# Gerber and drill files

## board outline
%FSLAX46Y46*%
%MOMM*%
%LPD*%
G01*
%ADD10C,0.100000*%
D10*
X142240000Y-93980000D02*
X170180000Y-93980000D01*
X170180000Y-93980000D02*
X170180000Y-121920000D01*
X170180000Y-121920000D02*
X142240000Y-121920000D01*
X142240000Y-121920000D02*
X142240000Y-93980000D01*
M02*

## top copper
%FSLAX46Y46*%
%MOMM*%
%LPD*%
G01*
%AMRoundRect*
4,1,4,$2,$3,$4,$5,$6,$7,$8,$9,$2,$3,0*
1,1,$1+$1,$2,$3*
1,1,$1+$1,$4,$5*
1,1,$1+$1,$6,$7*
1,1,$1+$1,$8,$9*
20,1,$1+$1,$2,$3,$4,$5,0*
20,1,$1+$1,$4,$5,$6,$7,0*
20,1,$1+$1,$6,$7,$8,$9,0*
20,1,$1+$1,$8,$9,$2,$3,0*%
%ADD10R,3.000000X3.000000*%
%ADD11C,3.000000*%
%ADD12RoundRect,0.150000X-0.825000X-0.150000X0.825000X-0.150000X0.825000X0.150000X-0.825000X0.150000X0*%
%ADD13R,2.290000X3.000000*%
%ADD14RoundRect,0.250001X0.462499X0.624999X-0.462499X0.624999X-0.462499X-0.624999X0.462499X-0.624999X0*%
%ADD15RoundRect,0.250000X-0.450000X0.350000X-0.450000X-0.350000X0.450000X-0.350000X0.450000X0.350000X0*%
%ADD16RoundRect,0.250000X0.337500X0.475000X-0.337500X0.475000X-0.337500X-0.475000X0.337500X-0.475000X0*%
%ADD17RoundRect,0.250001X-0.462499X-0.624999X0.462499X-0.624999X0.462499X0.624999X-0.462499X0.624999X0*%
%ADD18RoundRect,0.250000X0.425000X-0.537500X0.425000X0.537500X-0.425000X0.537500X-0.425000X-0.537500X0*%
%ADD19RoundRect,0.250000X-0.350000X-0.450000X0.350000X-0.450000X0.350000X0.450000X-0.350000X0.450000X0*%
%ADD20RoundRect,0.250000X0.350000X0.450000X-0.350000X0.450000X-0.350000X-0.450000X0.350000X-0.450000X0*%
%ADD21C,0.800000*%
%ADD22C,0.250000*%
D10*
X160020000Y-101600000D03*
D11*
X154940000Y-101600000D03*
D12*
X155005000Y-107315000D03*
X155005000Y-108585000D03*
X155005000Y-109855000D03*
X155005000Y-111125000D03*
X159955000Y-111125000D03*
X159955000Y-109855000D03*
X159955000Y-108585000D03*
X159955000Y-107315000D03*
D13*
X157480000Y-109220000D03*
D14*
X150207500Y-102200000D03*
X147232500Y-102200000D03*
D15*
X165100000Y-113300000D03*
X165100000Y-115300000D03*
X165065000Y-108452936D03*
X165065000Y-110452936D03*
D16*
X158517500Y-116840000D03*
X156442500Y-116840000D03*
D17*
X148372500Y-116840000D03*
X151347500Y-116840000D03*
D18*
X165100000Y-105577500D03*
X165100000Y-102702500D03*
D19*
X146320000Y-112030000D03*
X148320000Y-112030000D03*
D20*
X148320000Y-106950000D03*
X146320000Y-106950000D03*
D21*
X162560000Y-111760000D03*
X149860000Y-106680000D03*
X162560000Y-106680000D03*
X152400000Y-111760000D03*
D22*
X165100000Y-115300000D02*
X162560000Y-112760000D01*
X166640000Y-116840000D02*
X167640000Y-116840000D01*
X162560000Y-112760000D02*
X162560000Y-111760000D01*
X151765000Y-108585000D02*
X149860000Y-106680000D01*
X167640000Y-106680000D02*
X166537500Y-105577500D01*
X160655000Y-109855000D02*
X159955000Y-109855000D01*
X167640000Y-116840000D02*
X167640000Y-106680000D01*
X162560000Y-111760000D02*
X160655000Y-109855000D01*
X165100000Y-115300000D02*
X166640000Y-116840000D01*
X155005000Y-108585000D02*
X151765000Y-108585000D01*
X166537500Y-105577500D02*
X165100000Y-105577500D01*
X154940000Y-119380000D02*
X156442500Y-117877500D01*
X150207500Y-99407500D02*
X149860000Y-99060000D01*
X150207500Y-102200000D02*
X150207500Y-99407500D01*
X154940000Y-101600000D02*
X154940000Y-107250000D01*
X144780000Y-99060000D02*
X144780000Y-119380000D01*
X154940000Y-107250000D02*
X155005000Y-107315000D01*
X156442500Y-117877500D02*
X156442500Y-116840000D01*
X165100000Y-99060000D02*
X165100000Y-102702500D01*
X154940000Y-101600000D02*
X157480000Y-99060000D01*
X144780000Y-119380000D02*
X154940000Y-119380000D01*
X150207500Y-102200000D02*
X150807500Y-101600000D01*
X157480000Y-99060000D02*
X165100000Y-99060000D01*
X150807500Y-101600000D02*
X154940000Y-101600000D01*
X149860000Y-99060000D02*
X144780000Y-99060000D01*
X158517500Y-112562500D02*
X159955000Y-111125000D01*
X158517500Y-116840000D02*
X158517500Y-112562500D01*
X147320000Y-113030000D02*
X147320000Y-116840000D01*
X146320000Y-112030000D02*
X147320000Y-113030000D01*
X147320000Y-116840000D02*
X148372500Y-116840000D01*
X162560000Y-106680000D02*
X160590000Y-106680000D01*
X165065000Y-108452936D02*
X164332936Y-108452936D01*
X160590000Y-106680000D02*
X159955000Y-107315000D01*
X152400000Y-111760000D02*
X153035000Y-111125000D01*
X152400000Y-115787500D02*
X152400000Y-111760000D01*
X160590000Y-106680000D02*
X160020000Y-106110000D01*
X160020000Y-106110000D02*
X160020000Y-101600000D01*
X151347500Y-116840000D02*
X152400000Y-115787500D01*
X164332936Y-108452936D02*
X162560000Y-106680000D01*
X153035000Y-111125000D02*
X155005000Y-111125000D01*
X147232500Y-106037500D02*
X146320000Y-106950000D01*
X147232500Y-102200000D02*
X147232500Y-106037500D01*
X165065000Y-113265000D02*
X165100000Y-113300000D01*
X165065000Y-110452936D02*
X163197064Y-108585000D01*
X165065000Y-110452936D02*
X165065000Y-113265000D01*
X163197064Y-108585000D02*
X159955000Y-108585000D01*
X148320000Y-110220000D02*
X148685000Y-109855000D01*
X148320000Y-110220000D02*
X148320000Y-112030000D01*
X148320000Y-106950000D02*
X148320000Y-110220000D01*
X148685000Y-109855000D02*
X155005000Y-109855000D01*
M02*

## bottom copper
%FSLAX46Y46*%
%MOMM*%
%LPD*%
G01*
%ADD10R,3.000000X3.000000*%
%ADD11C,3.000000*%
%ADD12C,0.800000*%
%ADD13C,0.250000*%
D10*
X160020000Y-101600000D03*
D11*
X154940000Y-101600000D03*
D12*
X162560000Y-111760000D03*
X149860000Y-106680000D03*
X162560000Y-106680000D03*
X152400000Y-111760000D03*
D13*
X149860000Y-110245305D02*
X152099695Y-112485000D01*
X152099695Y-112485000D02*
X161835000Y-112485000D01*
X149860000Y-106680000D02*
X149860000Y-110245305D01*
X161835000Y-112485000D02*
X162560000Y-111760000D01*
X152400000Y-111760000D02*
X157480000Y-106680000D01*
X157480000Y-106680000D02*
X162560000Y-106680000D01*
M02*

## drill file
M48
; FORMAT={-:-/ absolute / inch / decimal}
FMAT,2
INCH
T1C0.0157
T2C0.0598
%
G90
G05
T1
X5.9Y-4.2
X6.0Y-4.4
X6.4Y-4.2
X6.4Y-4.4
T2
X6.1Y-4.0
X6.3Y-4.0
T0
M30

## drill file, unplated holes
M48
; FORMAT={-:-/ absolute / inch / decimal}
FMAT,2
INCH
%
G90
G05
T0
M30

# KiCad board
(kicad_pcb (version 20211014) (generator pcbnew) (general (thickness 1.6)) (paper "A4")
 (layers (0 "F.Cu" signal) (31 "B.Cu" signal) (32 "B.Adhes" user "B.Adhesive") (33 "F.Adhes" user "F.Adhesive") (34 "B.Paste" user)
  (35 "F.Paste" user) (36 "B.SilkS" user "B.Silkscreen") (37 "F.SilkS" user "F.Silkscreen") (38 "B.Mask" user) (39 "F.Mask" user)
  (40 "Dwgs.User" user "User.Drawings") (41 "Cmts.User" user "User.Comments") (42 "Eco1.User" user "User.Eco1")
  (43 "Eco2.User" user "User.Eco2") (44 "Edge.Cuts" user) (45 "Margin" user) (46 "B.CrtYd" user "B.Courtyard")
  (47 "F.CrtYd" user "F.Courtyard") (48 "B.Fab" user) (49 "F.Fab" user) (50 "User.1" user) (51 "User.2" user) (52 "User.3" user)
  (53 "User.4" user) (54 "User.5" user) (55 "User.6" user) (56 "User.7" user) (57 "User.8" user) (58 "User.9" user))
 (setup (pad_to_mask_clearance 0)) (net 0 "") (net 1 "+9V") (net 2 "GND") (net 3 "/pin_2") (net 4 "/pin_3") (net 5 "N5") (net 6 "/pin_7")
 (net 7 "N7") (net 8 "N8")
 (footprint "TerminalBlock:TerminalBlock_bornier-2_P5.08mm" (layer "F.Cu") (at 160.02 101.6 180)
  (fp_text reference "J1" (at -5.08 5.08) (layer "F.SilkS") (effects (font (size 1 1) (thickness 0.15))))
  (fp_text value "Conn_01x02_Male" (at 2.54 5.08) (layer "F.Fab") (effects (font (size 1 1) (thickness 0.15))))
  (pad "1" thru_hole rect (at 0 0 180) (size 3 3) (drill 1.52) (layers *.Cu *.Mask) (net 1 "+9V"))
  (pad "2" thru_hole circle (at 5.08 0 180) (size 3 3) (drill 1.52) (layers *.Cu *.Mask) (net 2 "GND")))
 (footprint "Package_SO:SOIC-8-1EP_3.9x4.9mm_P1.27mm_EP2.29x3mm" (layer "F.Cu") (at 157.48 109.22)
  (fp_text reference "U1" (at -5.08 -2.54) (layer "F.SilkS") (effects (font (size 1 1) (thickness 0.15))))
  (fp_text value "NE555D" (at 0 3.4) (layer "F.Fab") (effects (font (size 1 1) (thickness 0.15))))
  (pad "" smd roundrect (at -0.57 -0.75) (size 0.92 1.21) (layers "F.Paste") (roundrect_rratio 0.25))
  (pad "" smd roundrect (at -0.57 0.75) (size 0.92 1.21) (layers "F.Paste") (roundrect_rratio 0.25))
  (pad "" smd roundrect (at 0.57 -0.75) (size 0.92 1.21) (layers "F.Paste") (roundrect_rratio 0.25))
  (pad "" smd roundrect (at 0.57 0.75) (size 0.92 1.21) (layers "F.Paste") (roundrect_rratio 0.25))
  (pad "1" smd roundrect (at -2.475 -1.905) (size 1.95 0.6) (layers "F.Cu" "F.Paste" "F.Mask") (roundrect_rratio 0.25) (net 2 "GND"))
  (pad "2" smd roundrect (at -2.475 -0.635) (size 1.95 0.6) (layers "F.Cu" "F.Paste" "F.Mask") (roundrect_rratio 0.25) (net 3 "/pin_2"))
  (pad "3" smd roundrect (at -2.475 0.635) (size 1.95 0.6) (layers "F.Cu" "F.Paste" "F.Mask") (roundrect_rratio 0.25) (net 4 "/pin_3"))
  (pad "4" smd roundrect (at -2.475 1.905) (size 1.95 0.6) (layers "F.Cu" "F.Paste" "F.Mask") (roundrect_rratio 0.25) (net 1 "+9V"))
  (pad "5" smd roundrect (at 2.475 1.905) (size 1.95 0.6) (layers "F.Cu" "F.Paste" "F.Mask") (roundrect_rratio 0.25) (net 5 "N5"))
  (pad "6" smd roundrect (at 2.475 0.635) (size 1.95 0.6) (layers "F.Cu" "F.Paste" "F.Mask") (roundrect_rratio 0.25) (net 3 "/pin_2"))
  (pad "7" smd roundrect (at 2.475 -0.635) (size 1.95 0.6) (layers "F.Cu" "F.Paste" "F.Mask") (roundrect_rratio 0.25) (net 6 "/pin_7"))
  (pad "8" smd roundrect (at 2.475 -1.905) (size 1.95 0.6) (layers "F.Cu" "F.Paste" "F.Mask") (roundrect_rratio 0.25) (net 1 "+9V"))
  (pad "9" smd rect (at 0 0) (size 2.29 3) (layers "F.Cu" "F.Mask")))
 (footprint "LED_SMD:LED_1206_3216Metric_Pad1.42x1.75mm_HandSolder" (layer "F.Cu") (at 148.72 102.2 180)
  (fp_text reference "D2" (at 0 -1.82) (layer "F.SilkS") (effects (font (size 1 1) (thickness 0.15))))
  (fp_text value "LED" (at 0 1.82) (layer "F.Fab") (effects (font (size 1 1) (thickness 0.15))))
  (pad "1" smd roundrect (at -1.4875 0 180) (size 1.425 1.75) (layers "F.Cu" "F.Paste" "F.Mask") (roundrect_rratio 0.1754392982)
   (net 2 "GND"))
  (pad "2" smd roundrect (at 1.4875 0 180) (size 1.425 1.75) (layers "F.Cu" "F.Paste" "F.Mask") (roundrect_rratio 0.1754392982) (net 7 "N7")))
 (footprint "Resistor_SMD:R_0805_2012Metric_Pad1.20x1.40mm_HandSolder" (layer "F.Cu") (at 165.1 114.3 -90)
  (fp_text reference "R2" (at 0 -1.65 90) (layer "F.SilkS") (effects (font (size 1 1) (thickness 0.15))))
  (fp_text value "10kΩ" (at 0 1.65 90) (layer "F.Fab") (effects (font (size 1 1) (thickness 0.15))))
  (pad "1" smd roundrect (at -1 0 270) (size 1.2 1.4) (layers "F.Cu" "F.Paste" "F.Mask") (roundrect_rratio 0.2083333333) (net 6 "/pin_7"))
  (pad "2" smd roundrect (at 1 0 270) (size 1.2 1.4) (layers "F.Cu" "F.Paste" "F.Mask") (roundrect_rratio 0.2083333333) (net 3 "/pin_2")))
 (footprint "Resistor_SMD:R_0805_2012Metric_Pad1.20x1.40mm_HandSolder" (layer "F.Cu") (at 165.065 109.452936 -90)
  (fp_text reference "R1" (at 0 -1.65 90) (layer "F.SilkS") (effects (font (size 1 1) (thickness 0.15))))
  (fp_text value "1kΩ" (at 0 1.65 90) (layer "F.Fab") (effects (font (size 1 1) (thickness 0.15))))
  (pad "1" smd roundrect (at -1 0 270) (size 1.2 1.4) (layers "F.Cu" "F.Paste" "F.Mask") (roundrect_rratio 0.2083333333) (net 1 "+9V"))
  (pad "2" smd roundrect (at 1 0 270) (size 1.2 1.4) (layers "F.Cu" "F.Paste" "F.Mask") (roundrect_rratio 0.2083333333) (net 6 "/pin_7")))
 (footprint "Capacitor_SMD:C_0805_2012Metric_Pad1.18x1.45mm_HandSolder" (layer "F.Cu") (at 157.48 116.84 180)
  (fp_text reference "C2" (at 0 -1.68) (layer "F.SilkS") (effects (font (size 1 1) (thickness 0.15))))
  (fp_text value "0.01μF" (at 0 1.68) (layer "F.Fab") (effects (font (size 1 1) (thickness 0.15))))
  (pad "1" smd roundrect (at -1.0375 0 180) (size 1.175 1.45) (layers "F.Cu" "F.Paste" "F.Mask") (roundrect_rratio 0.2127659574)
   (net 5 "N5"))
  (pad "2" smd roundrect (at 1.0375 0 180) (size 1.175 1.45) (layers "F.Cu" "F.Paste" "F.Mask") (roundrect_rratio 0.2127659574)
   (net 2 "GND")))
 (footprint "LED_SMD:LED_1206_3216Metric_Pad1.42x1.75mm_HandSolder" (layer "F.Cu") (at 149.86 116.84)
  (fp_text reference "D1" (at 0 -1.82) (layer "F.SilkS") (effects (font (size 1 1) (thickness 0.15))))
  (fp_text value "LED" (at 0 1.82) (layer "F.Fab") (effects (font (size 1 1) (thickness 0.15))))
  (pad "1" smd roundrect (at -1.4875 0) (size 1.425 1.75) (layers "F.Cu" "F.Paste" "F.Mask") (roundrect_rratio 0.1754392982) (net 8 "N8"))
  (pad "2" smd roundrect (at 1.4875 0) (size 1.425 1.75) (layers "F.Cu" "F.Paste" "F.Mask") (roundrect_rratio 0.1754392982) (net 1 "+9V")))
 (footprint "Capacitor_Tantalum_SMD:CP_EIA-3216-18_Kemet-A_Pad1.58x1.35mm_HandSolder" (layer "F.Cu") (at 165.1 104.14 90)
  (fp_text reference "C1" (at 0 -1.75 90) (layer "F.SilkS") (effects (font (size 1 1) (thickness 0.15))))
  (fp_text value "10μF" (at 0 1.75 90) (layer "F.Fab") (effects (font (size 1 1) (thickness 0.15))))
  (pad "1" smd roundrect (at -1.4375 0 90) (size 1.575 1.35) (layers "F.Cu" "F.Paste" "F.Mask") (roundrect_rratio 0.1851851852)
   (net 3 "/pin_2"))
  (pad "2" smd roundrect (at 1.4375 0 90) (size 1.575 1.35) (layers "F.Cu" "F.Paste" "F.Mask") (roundrect_rratio 0.1851851852) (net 2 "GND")))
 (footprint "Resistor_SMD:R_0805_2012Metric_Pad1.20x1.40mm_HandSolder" (layer "F.Cu") (at 147.32 112.03)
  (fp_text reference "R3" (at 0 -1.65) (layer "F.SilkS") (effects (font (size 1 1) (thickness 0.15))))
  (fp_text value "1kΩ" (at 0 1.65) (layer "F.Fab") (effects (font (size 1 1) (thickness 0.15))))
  (pad "1" smd roundrect (at -1 0) (size 1.2 1.4) (layers "F.Cu" "F.Paste" "F.Mask") (roundrect_rratio 0.2083333333) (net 8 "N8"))
  (pad "2" smd roundrect (at 1 0) (size 1.2 1.4) (layers "F.Cu" "F.Paste" "F.Mask") (roundrect_rratio 0.2083333333) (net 4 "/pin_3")))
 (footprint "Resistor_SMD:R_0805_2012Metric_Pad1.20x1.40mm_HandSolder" (layer "F.Cu") (at 147.32 106.95 180)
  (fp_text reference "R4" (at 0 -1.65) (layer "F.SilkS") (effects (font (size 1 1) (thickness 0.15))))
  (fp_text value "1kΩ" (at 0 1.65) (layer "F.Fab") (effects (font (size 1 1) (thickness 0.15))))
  (pad "1" smd roundrect (at -1 0 180) (size 1.2 1.4) (layers "F.Cu" "F.Paste" "F.Mask") (roundrect_rratio 0.2083333333) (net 4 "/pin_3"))
  (pad "2" smd roundrect (at 1 0 180) (size 1.2 1.4) (layers "F.Cu" "F.Paste" "F.Mask") (roundrect_rratio 0.2083333333) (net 7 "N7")))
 (gr_rect (start 142.24 93.98) (end 170.18 121.92) (layer "Edge.Cuts") (width 0.1) (fill none))
 (segment (start 165.1 115.3) (end 162.56 112.76) (width 0.25) (layer "F.Cu") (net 3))
 (segment (start 166.64 116.84) (end 167.64 116.84) (width 0.25) (layer "F.Cu") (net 3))
 (segment (start 162.56 112.76) (end 162.56 111.76) (width 0.25) (layer "F.Cu") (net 3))
 (segment (start 151.765 108.585) (end 149.86 106.68) (width 0.25) (layer "F.Cu") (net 3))
 (segment (start 167.64 106.68) (end 166.5375 105.5775) (width 0.25) (layer "F.Cu") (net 3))
 (segment (start 160.655 109.855) (end 159.955 109.855) (width 0.25) (layer "F.Cu") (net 3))
 (segment (start 167.64 116.84) (end 167.64 106.68) (width 0.25) (layer "F.Cu") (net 3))
 (segment (start 162.56 111.76) (end 160.655 109.855) (width 0.25) (layer "F.Cu") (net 3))
 (segment (start 165.1 115.3) (end 166.64 116.84) (width 0.25) (layer "F.Cu") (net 3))
 (segment (start 155.005 108.585) (end 151.765 108.585) (width 0.25) (layer "F.Cu") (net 3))
 (segment (start 166.5375 105.5775) (end 165.1 105.5775) (width 0.25) (layer "F.Cu") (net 3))
 (via (at 162.56 111.76) (size 0.8) (drill 0.4) (layers "F.Cu" "B.Cu") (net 3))
 (via (at 149.86 106.68) (size 0.8) (drill 0.4) (layers "F.Cu" "B.Cu") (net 3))
 (segment (start 149.86 110.245305) (end 152.099695 112.485) (width 0.25) (layer "B.Cu") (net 3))
 (segment (start 152.099695 112.485) (end 161.835 112.485) (width 0.25) (layer "B.Cu") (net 3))
 (segment (start 149.86 106.68) (end 149.86 110.245305) (width 0.25) (layer "B.Cu") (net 3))
 (segment (start 161.835 112.485) (end 162.56 111.76) (width 0.25) (layer "B.Cu") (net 3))
 (segment (start 154.94 119.38) (end 156.4425 117.8775) (width 0.25) (layer "F.Cu") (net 2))
 (segment (start 150.2075 99.4075) (end 149.86 99.06) (width 0.25) (layer "F.Cu") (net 2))
 (segment (start 150.2075 102.2) (end 150.2075 99.4075) (width 0.25) (layer "F.Cu") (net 2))
 (segment (start 154.94 101.6) (end 154.94 107.25) (width 0.25) (layer "F.Cu") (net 2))
 (segment (start 144.78 99.06) (end 144.78 119.38) (width 0.25) (layer "F.Cu") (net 2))
 (segment (start 154.94 107.25) (end 155.005 107.315) (width 0.25) (layer "F.Cu") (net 2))
 (segment (start 156.4425 117.8775) (end 156.4425 116.84) (width 0.25) (layer "F.Cu") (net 2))
 (segment (start 165.1 99.06) (end 165.1 102.7025) (width 0.25) (layer "F.Cu") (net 2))
 (segment (start 154.94 101.6) (end 157.48 99.06) (width 0.25) (layer "F.Cu") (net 2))
 (segment (start 144.78 119.38) (end 154.94 119.38) (width 0.25) (layer "F.Cu") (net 2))
 (segment (start 150.2075 102.2) (end 150.8075 101.6) (width 0.25) (layer "F.Cu") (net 2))
 (segment (start 157.48 99.06) (end 165.1 99.06) (width 0.25) (layer "F.Cu") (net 2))
 (segment (start 150.8075 101.6) (end 154.94 101.6) (width 0.25) (layer "F.Cu") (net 2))
 (segment (start 149.86 99.06) (end 144.78 99.06) (width 0.25) (layer "F.Cu") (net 2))
 (segment (start 158.5175 112.5625) (end 159.955 111.125) (width 0.25) (layer "F.Cu") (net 5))
 (segment (start 158.5175 116.84) (end 158.5175 112.5625) (width 0.25) (layer "F.Cu") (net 5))
 (segment (start 147.32 113.03) (end 147.32 116.84) (width 0.25) (layer "F.Cu") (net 8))
 (segment (start 146.32 112.03) (end 147.32 113.03) (width 0.25) (layer "F.Cu") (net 8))
 (segment (start 147.32 116.84) (end 148.3725 116.84) (width 0.25) (layer "F.Cu") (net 8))
 (segment (start 162.56 106.68) (end 160.59 106.68) (width 0.25) (layer "F.Cu") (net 1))
 (segment (start 165.065 108.452936) (end 164.332936 108.452936) (width 0.25) (layer "F.Cu") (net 1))
 (segment (start 160.59 106.68) (end 159.955 107.315) (width 0.25) (layer "F.Cu") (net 1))
 (segment (start 152.4 111.76) (end 153.035 111.125) (width 0.25) (layer "F.Cu") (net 1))
 (segment (start 152.4 115.7875) (end 152.4 111.76) (width 0.25) (layer "F.Cu") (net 1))
 (segment (start 160.59 106.68) (end 160.02 106.11) (width 0.25) (layer "F.Cu") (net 1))
 (segment (start 160.02 106.11) (end 160.02 101.6) (width 0.25) (layer "F.Cu") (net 1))
 (segment (start 151.3475 116.84) (end 152.4 115.7875) (width 0.25) (layer "F.Cu") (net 1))
 (segment (start 164.332936 108.452936) (end 162.56 106.68) (width 0.25) (layer "F.Cu") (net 1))
 (segment (start 153.035 111.125) (end 155.005 111.125) (width 0.25) (layer "F.Cu") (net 1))
 (via (at 162.56 106.68) (size 0.8) (drill 0.4) (layers "F.Cu" "B.Cu") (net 1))
 (via (at 152.4 111.76) (size 0.8) (drill 0.4) (layers "F.Cu" "B.Cu") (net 1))
 (segment (start 152.4 111.76) (end 157.48 106.68) (width 0.25) (layer "B.Cu") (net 1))
 (segment (start 157.48 106.68) (end 162.56 106.68) (width 0.25) (layer "B.Cu") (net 1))
 (segment (start 147.2325 106.0375) (end 146.32 106.95) (width 0.25) (layer "F.Cu") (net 7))
 (segment (start 147.2325 102.2) (end 147.2325 106.0375) (width 0.25) (layer "F.Cu") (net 7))
 (segment (start 165.065 113.265) (end 165.1 113.3) (width 0.25) (layer "F.Cu") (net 6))
 (segment (start 165.065 110.452936) (end 163.197064 108.585) (width 0.25) (layer "F.Cu") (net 6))
 (segment (start 165.065 110.452936) (end 165.065 113.265) (width 0.25) (layer "F.Cu") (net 6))
 (segment (start 163.197064 108.585) (end 159.955 108.585) (width 0.25) (layer "F.Cu") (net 6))
 (segment (start 148.32 110.22) (end 148.685 109.855) (width 0.25) (layer "F.Cu") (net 4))
 (segment (start 148.32 110.22) (end 148.32 112.03) (width 0.25) (layer "F.Cu") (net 4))
 (segment (start 148.32 106.95) (end 148.32 110.22) (width 0.25) (layer "F.Cu") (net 4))
 (segment (start 148.685 109.855) (end 155.005 109.855) (width 0.25) (layer "F.Cu") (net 4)))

